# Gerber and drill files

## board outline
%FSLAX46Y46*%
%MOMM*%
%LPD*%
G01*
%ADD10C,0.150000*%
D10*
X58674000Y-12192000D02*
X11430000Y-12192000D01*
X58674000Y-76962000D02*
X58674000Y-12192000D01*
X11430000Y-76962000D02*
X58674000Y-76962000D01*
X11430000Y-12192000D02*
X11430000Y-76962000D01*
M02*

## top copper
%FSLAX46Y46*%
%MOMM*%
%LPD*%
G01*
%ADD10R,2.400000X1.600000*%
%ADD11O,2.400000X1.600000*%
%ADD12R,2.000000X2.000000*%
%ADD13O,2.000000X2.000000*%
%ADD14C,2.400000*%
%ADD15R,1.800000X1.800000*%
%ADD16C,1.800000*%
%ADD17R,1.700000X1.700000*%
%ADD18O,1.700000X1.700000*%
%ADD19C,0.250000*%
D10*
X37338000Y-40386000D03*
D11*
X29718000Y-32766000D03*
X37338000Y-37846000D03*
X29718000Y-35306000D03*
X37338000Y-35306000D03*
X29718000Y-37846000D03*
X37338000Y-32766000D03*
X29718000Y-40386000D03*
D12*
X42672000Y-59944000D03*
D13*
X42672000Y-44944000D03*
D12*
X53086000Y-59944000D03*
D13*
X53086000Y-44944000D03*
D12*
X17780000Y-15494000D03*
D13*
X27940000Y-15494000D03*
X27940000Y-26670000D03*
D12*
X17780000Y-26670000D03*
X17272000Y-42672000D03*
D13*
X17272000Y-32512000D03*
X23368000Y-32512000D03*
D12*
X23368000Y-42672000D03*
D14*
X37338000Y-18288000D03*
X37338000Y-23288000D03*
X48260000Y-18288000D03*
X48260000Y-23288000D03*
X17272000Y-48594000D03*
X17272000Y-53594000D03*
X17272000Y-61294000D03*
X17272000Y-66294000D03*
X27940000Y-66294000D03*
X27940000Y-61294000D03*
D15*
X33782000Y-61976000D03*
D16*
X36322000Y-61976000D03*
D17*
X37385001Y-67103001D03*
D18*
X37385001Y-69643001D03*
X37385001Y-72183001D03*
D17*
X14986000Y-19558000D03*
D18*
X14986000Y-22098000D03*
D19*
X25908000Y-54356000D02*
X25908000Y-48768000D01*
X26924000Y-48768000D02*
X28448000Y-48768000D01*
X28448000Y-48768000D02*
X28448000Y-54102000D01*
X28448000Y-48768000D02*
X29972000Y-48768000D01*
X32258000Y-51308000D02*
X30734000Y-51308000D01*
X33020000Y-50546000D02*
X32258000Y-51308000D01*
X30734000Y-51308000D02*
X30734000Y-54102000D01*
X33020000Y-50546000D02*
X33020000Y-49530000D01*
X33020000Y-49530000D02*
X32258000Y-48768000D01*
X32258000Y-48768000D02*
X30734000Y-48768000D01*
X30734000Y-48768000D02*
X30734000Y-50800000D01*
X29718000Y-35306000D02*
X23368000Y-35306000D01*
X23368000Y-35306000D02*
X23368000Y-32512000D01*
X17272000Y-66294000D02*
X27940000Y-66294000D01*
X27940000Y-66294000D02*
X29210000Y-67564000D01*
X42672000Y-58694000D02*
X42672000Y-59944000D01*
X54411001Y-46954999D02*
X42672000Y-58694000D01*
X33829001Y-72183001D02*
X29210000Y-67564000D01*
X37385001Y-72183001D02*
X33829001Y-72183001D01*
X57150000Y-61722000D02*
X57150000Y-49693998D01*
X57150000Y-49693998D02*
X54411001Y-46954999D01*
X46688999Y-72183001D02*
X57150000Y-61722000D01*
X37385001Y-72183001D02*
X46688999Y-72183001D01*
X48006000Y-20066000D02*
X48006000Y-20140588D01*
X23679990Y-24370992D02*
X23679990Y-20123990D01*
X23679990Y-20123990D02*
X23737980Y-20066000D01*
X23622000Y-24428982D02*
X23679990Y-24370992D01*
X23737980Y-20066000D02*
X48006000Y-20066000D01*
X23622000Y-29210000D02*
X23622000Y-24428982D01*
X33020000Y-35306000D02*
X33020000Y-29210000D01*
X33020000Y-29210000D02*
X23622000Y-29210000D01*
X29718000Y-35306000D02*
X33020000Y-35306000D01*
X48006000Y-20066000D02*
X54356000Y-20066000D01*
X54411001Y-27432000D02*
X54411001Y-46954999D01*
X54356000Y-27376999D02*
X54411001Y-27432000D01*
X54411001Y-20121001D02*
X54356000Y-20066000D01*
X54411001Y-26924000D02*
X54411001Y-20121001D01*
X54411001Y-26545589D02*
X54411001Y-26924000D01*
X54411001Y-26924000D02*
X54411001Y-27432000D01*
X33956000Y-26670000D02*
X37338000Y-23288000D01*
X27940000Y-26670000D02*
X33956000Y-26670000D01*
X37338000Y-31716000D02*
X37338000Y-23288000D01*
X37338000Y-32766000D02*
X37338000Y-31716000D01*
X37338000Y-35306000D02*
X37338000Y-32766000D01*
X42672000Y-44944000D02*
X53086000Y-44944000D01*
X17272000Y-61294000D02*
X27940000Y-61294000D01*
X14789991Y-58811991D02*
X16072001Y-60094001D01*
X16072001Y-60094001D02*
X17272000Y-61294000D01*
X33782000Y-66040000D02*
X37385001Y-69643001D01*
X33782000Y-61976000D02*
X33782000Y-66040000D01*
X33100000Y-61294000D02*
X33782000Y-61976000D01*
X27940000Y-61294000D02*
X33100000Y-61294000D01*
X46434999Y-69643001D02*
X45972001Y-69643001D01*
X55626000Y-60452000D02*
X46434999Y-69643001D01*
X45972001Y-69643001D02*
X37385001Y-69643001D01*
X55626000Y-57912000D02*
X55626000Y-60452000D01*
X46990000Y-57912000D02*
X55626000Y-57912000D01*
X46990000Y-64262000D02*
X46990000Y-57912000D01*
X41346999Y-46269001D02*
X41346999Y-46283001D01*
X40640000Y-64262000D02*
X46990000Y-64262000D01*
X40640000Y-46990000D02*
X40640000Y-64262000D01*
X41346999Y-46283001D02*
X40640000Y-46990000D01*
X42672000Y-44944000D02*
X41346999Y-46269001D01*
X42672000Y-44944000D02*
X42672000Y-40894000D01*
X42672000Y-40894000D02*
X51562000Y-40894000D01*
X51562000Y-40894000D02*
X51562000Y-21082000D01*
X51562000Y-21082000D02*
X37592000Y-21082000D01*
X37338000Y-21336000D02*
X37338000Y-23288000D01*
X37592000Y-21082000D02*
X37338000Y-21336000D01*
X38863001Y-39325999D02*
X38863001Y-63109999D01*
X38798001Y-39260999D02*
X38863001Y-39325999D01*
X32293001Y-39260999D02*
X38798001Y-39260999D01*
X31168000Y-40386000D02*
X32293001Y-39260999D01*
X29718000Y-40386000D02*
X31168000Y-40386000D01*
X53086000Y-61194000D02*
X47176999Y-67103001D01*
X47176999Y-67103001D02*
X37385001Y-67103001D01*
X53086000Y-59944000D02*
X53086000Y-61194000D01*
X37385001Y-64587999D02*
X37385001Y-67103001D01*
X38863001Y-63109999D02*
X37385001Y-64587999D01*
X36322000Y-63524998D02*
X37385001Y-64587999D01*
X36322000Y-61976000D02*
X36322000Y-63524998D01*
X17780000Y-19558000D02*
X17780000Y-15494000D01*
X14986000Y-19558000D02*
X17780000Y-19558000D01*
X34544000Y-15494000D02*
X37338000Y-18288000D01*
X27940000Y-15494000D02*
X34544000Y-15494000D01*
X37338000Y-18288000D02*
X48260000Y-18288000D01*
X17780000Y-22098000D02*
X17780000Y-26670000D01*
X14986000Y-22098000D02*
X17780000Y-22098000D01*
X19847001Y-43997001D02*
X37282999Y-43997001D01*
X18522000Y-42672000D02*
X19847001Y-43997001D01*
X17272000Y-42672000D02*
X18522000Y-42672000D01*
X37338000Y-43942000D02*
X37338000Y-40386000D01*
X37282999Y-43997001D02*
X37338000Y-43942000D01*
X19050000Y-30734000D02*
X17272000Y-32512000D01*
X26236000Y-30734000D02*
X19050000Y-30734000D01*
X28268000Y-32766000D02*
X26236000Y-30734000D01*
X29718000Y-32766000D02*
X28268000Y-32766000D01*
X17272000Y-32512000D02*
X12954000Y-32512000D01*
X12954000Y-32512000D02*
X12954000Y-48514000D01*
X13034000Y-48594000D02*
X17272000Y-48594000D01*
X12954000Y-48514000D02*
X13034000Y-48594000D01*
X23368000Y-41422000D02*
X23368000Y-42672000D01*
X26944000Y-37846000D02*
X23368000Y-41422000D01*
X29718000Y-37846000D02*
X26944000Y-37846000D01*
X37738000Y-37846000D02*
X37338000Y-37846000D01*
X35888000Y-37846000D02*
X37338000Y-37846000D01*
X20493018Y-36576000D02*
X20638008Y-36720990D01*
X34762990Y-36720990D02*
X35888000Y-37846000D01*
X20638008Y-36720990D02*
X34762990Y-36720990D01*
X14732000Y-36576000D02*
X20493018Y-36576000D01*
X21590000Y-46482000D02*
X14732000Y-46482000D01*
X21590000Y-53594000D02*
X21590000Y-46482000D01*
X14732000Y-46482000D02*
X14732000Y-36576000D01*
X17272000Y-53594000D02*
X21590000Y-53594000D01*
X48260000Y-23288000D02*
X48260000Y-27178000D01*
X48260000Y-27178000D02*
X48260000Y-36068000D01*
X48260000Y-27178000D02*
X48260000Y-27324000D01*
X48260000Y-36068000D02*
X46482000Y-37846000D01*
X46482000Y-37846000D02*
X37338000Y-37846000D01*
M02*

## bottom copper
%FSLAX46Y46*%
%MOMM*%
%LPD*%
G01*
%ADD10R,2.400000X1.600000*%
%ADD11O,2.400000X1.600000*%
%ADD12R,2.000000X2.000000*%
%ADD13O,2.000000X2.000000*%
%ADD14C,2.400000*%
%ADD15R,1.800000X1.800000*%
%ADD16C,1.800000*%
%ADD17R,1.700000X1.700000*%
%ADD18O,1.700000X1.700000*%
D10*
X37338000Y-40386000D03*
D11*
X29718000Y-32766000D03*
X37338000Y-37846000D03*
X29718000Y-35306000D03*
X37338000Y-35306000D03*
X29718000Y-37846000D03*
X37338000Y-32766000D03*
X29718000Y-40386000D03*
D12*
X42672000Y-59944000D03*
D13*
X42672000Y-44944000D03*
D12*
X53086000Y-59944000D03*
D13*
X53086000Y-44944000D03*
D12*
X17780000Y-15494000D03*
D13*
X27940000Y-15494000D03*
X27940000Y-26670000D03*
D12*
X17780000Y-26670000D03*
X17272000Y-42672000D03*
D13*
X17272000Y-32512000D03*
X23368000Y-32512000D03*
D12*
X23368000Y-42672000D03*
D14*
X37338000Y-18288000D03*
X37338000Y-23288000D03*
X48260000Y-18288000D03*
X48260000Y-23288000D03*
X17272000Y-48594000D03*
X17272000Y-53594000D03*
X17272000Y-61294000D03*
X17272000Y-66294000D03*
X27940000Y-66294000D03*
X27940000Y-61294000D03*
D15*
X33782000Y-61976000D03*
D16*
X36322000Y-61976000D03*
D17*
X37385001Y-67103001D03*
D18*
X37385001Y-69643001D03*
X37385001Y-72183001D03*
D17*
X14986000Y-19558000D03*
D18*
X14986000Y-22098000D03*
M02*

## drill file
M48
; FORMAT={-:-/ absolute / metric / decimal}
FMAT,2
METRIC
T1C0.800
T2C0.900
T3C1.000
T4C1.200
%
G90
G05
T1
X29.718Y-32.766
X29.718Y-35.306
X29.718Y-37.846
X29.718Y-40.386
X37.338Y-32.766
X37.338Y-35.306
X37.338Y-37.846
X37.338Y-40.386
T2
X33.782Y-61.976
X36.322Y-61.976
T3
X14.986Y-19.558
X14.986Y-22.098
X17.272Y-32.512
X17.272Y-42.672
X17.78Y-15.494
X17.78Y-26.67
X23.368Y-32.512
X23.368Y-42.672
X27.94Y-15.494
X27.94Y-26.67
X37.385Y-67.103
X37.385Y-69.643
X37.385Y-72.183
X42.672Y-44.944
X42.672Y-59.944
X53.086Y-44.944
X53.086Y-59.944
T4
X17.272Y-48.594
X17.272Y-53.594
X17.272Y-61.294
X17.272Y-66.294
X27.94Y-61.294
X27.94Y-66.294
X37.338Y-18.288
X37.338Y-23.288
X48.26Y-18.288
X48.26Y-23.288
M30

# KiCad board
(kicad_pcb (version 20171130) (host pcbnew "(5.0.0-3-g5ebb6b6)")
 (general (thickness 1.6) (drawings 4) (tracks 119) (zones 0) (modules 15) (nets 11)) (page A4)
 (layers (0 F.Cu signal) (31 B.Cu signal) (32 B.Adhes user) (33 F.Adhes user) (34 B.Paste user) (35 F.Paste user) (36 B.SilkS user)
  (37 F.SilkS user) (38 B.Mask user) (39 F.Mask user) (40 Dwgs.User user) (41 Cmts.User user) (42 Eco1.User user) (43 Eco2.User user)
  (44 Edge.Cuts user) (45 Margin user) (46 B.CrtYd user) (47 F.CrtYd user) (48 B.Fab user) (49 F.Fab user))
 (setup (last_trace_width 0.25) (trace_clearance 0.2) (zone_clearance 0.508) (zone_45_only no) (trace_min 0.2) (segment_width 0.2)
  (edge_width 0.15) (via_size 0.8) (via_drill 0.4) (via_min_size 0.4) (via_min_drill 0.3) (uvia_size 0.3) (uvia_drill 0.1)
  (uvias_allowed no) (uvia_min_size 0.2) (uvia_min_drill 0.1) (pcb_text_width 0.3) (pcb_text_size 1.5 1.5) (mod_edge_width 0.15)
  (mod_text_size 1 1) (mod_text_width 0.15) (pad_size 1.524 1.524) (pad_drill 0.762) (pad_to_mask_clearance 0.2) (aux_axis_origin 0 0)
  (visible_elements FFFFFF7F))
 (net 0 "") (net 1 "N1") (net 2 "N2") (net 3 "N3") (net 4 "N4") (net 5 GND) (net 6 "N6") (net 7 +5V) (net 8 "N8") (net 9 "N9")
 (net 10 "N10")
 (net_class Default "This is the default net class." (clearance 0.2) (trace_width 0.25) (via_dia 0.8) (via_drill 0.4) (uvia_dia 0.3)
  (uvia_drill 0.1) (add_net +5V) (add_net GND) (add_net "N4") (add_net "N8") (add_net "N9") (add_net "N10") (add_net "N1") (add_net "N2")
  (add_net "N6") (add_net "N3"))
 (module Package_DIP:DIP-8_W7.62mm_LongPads (layer F.Cu) (at 37.338 40.386 180)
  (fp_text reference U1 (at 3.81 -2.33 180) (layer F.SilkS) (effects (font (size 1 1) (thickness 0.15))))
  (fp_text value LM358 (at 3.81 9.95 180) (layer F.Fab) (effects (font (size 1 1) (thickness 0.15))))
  (pad 1 thru_hole rect (at 0 0 180) (size 2.4 1.6) (drill 0.8) (layers *.Cu *.Mask) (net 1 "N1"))
  (pad 5 thru_hole oval (at 7.62 7.62 180) (size 2.4 1.6) (drill 0.8) (layers *.Cu *.Mask) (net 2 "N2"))
  (pad 2 thru_hole oval (at 0 2.54 180) (size 2.4 1.6) (drill 0.8) (layers *.Cu *.Mask) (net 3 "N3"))
  (pad 6 thru_hole oval (at 7.62 5.08 180) (size 2.4 1.6) (drill 0.8) (layers *.Cu *.Mask) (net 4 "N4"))
  (pad 3 thru_hole oval (at 0 5.08 180) (size 2.4 1.6) (drill 0.8) (layers *.Cu *.Mask) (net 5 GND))
  (pad 7 thru_hole oval (at 7.62 2.54 180) (size 2.4 1.6) (drill 0.8) (layers *.Cu *.Mask) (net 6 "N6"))
  (pad 4 thru_hole oval (at 0 7.62 180) (size 2.4 1.6) (drill 0.8) (layers *.Cu *.Mask) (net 5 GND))
  (pad 8 thru_hole oval (at 7.62 0 180) (size 2.4 1.6) (drill 0.8) (layers *.Cu *.Mask) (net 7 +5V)))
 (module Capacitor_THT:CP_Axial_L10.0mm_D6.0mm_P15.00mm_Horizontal (layer F.Cu) (at 42.672 59.944 90)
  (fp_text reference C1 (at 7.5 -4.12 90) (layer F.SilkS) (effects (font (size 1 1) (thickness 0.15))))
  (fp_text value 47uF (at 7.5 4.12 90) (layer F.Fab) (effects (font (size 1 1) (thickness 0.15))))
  (pad 1 thru_hole rect (at 0 0 90) (size 2 2) (drill 1) (layers *.Cu *.Mask) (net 4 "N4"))
  (pad 2 thru_hole oval (at 15 0 90) (size 2 2) (drill 1) (layers *.Cu *.Mask) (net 5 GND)))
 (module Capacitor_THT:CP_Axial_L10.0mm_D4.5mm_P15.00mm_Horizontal (layer F.Cu) (at 53.086 59.944 90)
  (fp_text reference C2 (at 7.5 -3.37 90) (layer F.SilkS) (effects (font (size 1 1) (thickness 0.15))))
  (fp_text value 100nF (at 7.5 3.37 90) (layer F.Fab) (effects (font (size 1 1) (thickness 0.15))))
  (pad 1 thru_hole rect (at 0 0 90) (size 2 2) (drill 1) (layers *.Cu *.Mask) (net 7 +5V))
  (pad 2 thru_hole oval (at 15 0 90) (size 2 2) (drill 1) (layers *.Cu *.Mask) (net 5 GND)))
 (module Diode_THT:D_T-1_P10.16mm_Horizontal (layer F.Cu) (at 17.78 15.494)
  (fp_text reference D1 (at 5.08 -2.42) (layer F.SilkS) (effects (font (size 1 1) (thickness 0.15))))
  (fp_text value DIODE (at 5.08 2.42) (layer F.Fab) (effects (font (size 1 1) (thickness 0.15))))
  (pad 1 thru_hole rect (at 0 0) (size 2 2) (drill 1) (layers *.Cu *.Mask) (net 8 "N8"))
  (pad 2 thru_hole oval (at 10.16 0) (size 2 2) (drill 1) (layers *.Cu *.Mask) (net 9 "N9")))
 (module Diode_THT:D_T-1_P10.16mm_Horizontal (layer F.Cu) (at 17.78 26.67)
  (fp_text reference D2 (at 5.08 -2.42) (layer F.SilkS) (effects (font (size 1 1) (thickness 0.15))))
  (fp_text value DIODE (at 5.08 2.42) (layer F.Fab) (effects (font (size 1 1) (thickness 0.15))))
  (pad 2 thru_hole oval (at 10.16 0) (size 2 2) (drill 1) (layers *.Cu *.Mask) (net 5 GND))
  (pad 1 thru_hole rect (at 0 0) (size 2 2) (drill 1) (layers *.Cu *.Mask) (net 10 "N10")))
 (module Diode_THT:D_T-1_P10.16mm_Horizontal (layer F.Cu) (at 17.272 42.672 90)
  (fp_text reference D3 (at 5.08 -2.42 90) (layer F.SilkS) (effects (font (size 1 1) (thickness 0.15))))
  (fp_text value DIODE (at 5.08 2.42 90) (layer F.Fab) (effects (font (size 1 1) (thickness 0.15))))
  (pad 1 thru_hole rect (at 0 0 90) (size 2 2) (drill 1) (layers *.Cu *.Mask) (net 1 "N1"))
  (pad 2 thru_hole oval (at 10.16 0 90) (size 2 2) (drill 1) (layers *.Cu *.Mask) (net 2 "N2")))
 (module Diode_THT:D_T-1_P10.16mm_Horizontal (layer F.Cu) (at 23.368 42.672 90)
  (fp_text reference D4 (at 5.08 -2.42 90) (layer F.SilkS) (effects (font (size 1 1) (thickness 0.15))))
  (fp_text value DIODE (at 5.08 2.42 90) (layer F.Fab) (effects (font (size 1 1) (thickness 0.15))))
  (pad 2 thru_hole oval (at 10.16 0 90) (size 2 2) (drill 1) (layers *.Cu *.Mask) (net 4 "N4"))
  (pad 1 thru_hole rect (at 0 0 90) (size 2 2) (drill 1) (layers *.Cu *.Mask) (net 6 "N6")))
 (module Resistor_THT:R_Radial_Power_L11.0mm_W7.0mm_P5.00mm (layer F.Cu) (at 37.338 18.288 270)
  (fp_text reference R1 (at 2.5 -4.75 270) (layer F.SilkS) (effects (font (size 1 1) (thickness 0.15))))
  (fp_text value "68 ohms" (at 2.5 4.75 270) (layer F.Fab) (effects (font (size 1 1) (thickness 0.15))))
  (pad 1 thru_hole circle (at 0 0 270) (size 2.4 2.4) (drill 1.2) (layers *.Cu *.Mask) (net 9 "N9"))
  (pad 2 thru_hole circle (at 5 0 270) (size 2.4 2.4) (drill 1.2) (layers *.Cu *.Mask) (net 5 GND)))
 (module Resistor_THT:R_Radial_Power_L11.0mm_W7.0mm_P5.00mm (layer F.Cu) (at 48.26 23.288 90)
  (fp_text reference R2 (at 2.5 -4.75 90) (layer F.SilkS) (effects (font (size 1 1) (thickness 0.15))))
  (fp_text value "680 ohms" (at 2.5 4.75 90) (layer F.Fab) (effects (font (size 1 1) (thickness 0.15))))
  (pad 2 thru_hole circle (at 5 0 90) (size 2.4 2.4) (drill 1.2) (layers *.Cu *.Mask) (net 9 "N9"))
  (pad 1 thru_hole circle (at 0 0 90) (size 2.4 2.4) (drill 1.2) (layers *.Cu *.Mask) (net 3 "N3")))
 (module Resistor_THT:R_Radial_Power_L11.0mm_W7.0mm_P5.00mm (layer F.Cu) (at 17.272 48.594 270)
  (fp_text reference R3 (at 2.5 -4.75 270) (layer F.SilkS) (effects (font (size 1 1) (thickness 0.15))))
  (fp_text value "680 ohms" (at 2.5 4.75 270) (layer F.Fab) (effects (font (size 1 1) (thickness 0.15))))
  (pad 1 thru_hole circle (at 0 0 270) (size 2.4 2.4) (drill 1.2) (layers *.Cu *.Mask) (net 2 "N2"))
  (pad 2 thru_hole circle (at 5 0 270) (size 2.4 2.4) (drill 1.2) (layers *.Cu *.Mask) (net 3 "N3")))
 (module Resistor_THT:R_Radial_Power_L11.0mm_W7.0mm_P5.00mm (layer F.Cu) (at 17.272 66.294 90)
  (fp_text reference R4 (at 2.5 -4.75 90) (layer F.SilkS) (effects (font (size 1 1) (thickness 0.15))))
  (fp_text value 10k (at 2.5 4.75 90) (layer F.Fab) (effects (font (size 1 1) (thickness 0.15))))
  (pad 2 thru_hole circle (at 5 0 90) (size 2.4 2.4) (drill 1.2) (layers *.Cu *.Mask) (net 5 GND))
  (pad 1 thru_hole circle (at 0 0 90) (size 2.4 2.4) (drill 1.2) (layers *.Cu *.Mask) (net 4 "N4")))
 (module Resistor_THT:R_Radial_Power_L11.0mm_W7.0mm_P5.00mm (layer F.Cu) (at 27.94 66.294 90)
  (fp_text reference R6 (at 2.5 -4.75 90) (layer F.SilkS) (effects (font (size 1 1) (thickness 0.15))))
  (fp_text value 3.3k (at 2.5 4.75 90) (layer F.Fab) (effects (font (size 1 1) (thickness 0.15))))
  (pad 1 thru_hole circle (at 0 0 90) (size 2.4 2.4) (drill 1.2) (layers *.Cu *.Mask) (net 4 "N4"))
  (pad 2 thru_hole circle (at 5 0 90) (size 2.4 2.4) (drill 1.2) (layers *.Cu *.Mask) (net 5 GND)))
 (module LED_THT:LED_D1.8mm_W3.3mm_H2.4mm (layer F.Cu) (at 33.782 61.976)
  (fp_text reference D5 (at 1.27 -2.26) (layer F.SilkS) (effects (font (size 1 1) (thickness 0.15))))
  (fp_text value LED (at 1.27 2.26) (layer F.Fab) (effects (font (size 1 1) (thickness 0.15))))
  (pad 1 thru_hole rect (at 0 0) (size 1.8 1.8) (drill 0.9) (layers *.Cu *.Mask) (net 5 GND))
  (pad 2 thru_hole circle (at 2.54 0) (size 1.8 1.8) (drill 0.9) (layers *.Cu *.Mask) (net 7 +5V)))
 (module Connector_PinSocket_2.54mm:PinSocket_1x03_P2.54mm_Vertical (layer F.Cu) (at 37.385001 67.103001)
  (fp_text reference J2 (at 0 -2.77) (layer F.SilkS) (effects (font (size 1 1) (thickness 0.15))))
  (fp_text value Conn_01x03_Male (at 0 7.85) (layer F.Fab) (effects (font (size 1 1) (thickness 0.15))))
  (pad 1 thru_hole rect (at 0 0) (size 1.7 1.7) (drill 1) (layers *.Cu *.Mask) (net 7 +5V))
  (pad 2 thru_hole oval (at 0 2.54) (size 1.7 1.7) (drill 1) (layers *.Cu *.Mask) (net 5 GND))
  (pad 3 thru_hole oval (at 0 5.08) (size 1.7 1.7) (drill 1) (layers *.Cu *.Mask) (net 4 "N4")))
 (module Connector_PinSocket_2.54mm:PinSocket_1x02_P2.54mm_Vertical (layer F.Cu) (at 14.986 19.558)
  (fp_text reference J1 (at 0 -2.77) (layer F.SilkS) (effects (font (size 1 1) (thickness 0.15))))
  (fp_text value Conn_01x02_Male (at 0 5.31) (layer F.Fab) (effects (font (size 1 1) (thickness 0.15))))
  (pad 1 thru_hole rect (at 0 0) (size 1.7 1.7) (drill 1) (layers *.Cu *.Mask) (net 8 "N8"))
  (pad 2 thru_hole oval (at 0 2.54) (size 1.7 1.7) (drill 1) (layers *.Cu *.Mask) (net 10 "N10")))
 (gr_line (start 58.674 12.192) (end 11.43 12.192) (layer Edge.Cuts) (width 0.15))
 (gr_line (start 58.674 76.962) (end 58.674 12.192) (layer Edge.Cuts) (width 0.15))
 (gr_line (start 11.43 76.962) (end 58.674 76.962) (layer Edge.Cuts) (width 0.15))
 (gr_line (start 11.43 12.192) (end 11.43 76.962) (layer Edge.Cuts) (width 0.15))
 (segment (start 25.908 54.356) (end 25.908 48.768) (width 0.25) (layer F.Cu) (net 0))
 (segment (start 26.924 48.768) (end 28.448 48.768) (width 0.25) (layer F.Cu) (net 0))
 (segment (start 28.448 48.768) (end 28.448 54.102) (width 0.25) (layer F.Cu) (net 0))
 (segment (start 28.448 48.768) (end 29.972 48.768) (width 0.25) (layer F.Cu) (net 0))
 (segment (start 32.258 51.308) (end 30.734 51.308) (width 0.25) (layer F.Cu) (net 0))
 (segment (start 33.02 50.546) (end 32.258 51.308) (width 0.25) (layer F.Cu) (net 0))
 (segment (start 30.734 51.308) (end 30.734 54.102) (width 0.25) (layer F.Cu) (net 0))
 (segment (start 33.02 50.546) (end 33.02 49.53) (width 0.25) (layer F.Cu) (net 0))
 (segment (start 33.02 49.53) (end 32.258 48.768) (width 0.25) (layer F.Cu) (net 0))
 (segment (start 32.258 48.768) (end 30.734 48.768) (width 0.25) (layer F.Cu) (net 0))
 (segment (start 30.734 48.768) (end 30.734 50.8) (width 0.25) (layer F.Cu) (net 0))
 (segment (start 29.718 35.306) (end 23.368 35.306) (width 0.25) (layer F.Cu) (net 4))
 (segment (start 23.368 35.306) (end 23.368 32.512) (width 0.25) (layer F.Cu) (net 4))
 (segment (start 17.272 66.294) (end 27.94 66.294) (width 0.25) (layer F.Cu) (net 4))
 (segment (start 27.94 66.294) (end 29.21 67.564) (width 0.25) (layer F.Cu) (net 4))
 (segment (start 42.672 58.694) (end 42.672 59.944) (width 0.25) (layer F.Cu) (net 4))
 (segment (start 54.411001 46.954999) (end 42.672 58.694) (width 0.25) (layer F.Cu) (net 4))
 (segment (start 33.829001 72.183001) (end 29.21 67.564) (width 0.25) (layer F.Cu) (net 4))
 (segment (start 37.385001 72.183001) (end 33.829001 72.183001) (width 0.25) (layer F.Cu) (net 4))
 (segment (start 57.15 61.722) (end 57.15 49.693998) (width 0.25) (layer F.Cu) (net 4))
 (segment (start 57.15 49.693998) (end 54.411001 46.954999) (width 0.25) (layer F.Cu) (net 4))
 (segment (start 46.688999 72.183001) (end 57.15 61.722) (width 0.25) (layer F.Cu) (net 4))
 (segment (start 37.385001 72.183001) (end 46.688999 72.183001) (width 0.25) (layer F.Cu) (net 4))
 (segment (start 48.006 20.066) (end 48.006 20.140588) (width 0.25) (layer F.Cu) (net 4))
 (segment (start 23.67999 24.370992) (end 23.67999 20.12399) (width 0.25) (layer F.Cu) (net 4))
 (segment (start 23.67999 20.12399) (end 23.73798 20.066) (width 0.25) (layer F.Cu) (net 4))
 (segment (start 23.622 24.428982) (end 23.67999 24.370992) (width 0.25) (layer F.Cu) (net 4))
 (segment (start 23.73798 20.066) (end 48.006 20.066) (width 0.25) (layer F.Cu) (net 4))
 (segment (start 23.622 29.21) (end 23.622 24.428982) (width 0.25) (layer F.Cu) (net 4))
 (segment (start 33.02 35.306) (end 33.02 29.21) (width 0.25) (layer F.Cu) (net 4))
 (segment (start 33.02 29.21) (end 23.622 29.21) (width 0.25) (layer F.Cu) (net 4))
 (segment (start 29.718 35.306) (end 33.02 35.306) (width 0.25) (layer F.Cu) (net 4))
 (segment (start 48.006 20.066) (end 54.356 20.066) (width 0.25) (layer F.Cu) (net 4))
 (segment (start 54.411001 27.432) (end 54.411001 46.954999) (width 0.25) (layer F.Cu) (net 4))
 (segment (start 54.356 27.376999) (end 54.411001 27.432) (width 0.25) (layer F.Cu) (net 4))
 (segment (start 54.411001 20.121001) (end 54.356 20.066) (width 0.25) (layer F.Cu) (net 4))
 (segment (start 54.411001 26.924) (end 54.411001 20.121001) (width 0.25) (layer F.Cu) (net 4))
 (segment (start 54.411001 26.545589) (end 54.411001 26.924) (width 0.25) (layer F.Cu) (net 4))
 (segment (start 54.411001 26.924) (end 54.411001 27.432) (width 0.25) (layer F.Cu) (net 4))
 (segment (start 33.956 26.67) (end 37.338 23.288) (width 0.25) (layer F.Cu) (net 5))
 (segment (start 27.94 26.67) (end 33.956 26.67) (width 0.25) (layer F.Cu) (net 5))
 (segment (start 37.338 31.716) (end 37.338 23.288) (width 0.25) (layer F.Cu) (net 5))
 (segment (start 37.338 32.766) (end 37.338 31.716) (width 0.25) (layer F.Cu) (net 5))
 (segment (start 37.338 35.306) (end 37.338 32.766) (width 0.25) (layer F.Cu) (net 5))
 (segment (start 42.672 44.944) (end 53.086 44.944) (width 0.25) (layer F.Cu) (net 5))
 (segment (start 17.272 61.294) (end 27.94 61.294) (width 0.25) (layer F.Cu) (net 5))
 (segment (start 14.789991 58.811991) (end 16.072001 60.094001) (width 0.25) (layer F.Cu) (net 5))
 (segment (start 16.072001 60.094001) (end 17.272 61.294) (width 0.25) (layer F.Cu) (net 5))
 (segment (start 33.782 66.04) (end 37.385001 69.643001) (width 0.25) (layer F.Cu) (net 5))
 (segment (start 33.782 61.976) (end 33.782 66.04) (width 0.25) (layer F.Cu) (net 5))
 (segment (start 33.1 61.294) (end 33.782 61.976) (width 0.25) (layer F.Cu) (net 5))
 (segment (start 27.94 61.294) (end 33.1 61.294) (width 0.25) (layer F.Cu) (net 5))
 (segment (start 46.434999 69.643001) (end 45.972001 69.643001) (width 0.25) (layer F.Cu) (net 5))
 (segment (start 55.626 60.452) (end 46.434999 69.643001) (width 0.25) (layer F.Cu) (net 5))
 (segment (start 45.972001 69.643001) (end 37.385001 69.643001) (width 0.25) (layer F.Cu) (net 5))
 (segment (start 55.626 57.912) (end 55.626 60.452) (width 0.25) (layer F.Cu) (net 5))
 (segment (start 46.99 57.912) (end 55.626 57.912) (width 0.25) (layer F.Cu) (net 5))
 (segment (start 46.99 64.262) (end 46.99 57.912) (width 0.25) (layer F.Cu) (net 5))
 (segment (start 41.346999 46.269001) (end 41.346999 46.283001) (width 0.25) (layer F.Cu) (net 5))
 (segment (start 40.64 64.262) (end 46.99 64.262) (width 0.25) (layer F.Cu) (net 5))
 (segment (start 40.64 46.99) (end 40.64 64.262) (width 0.25) (layer F.Cu) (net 5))
 (segment (start 41.346999 46.283001) (end 40.64 46.99) (width 0.25) (layer F.Cu) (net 5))
 (segment (start 42.672 44.944) (end 41.346999 46.269001) (width 0.25) (layer F.Cu) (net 5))
 (segment (start 42.672 44.944) (end 42.672 40.894) (width 0.25) (layer F.Cu) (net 5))
 (segment (start 42.672 40.894) (end 51.562 40.894) (width 0.25) (layer F.Cu) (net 5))
 (segment (start 51.562 40.894) (end 51.562 21.082) (width 0.25) (layer F.Cu) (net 5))
 (segment (start 51.562 21.082) (end 37.592 21.082) (width 0.25) (layer F.Cu) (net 5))
 (segment (start 37.338 21.336) (end 37.338 23.288) (width 0.25) (layer F.Cu) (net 5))
 (segment (start 37.592 21.082) (end 37.338 21.336) (width 0.25) (layer F.Cu) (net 5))
 (segment (start 38.863001 39.325999) (end 38.863001 63.109999) (width 0.25) (layer F.Cu) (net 7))
 (segment (start 38.798001 39.260999) (end 38.863001 39.325999) (width 0.25) (layer F.Cu) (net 7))
 (segment (start 32.293001 39.260999) (end 38.798001 39.260999) (width 0.25) (layer F.Cu) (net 7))
 (segment (start 31.168 40.386) (end 32.293001 39.260999) (width 0.25) (layer F.Cu) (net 7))
 (segment (start 29.718 40.386) (end 31.168 40.386) (width 0.25) (layer F.Cu) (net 7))
 (segment (start 53.086 61.194) (end 47.176999 67.103001) (width 0.25) (layer F.Cu) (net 7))
 (segment (start 47.176999 67.103001) (end 37.385001 67.103001) (width 0.25) (layer F.Cu) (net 7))
 (segment (start 53.086 59.944) (end 53.086 61.194) (width 0.25) (layer F.Cu) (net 7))
 (segment (start 37.385001 64.587999) (end 37.385001 67.103001) (width 0.25) (layer F.Cu) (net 7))
 (segment (start 38.863001 63.109999) (end 37.385001 64.587999) (width 0.25) (layer F.Cu) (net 7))
 (segment (start 36.322 63.524998) (end 37.385001 64.587999) (width 0.25) (layer F.Cu) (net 7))
 (segment (start 36.322 61.976) (end 36.322 63.524998) (width 0.25) (layer F.Cu) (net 7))
 (segment (start 17.78 19.558) (end 17.78 15.494) (width 0.25) (layer F.Cu) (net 8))
 (segment (start 14.986 19.558) (end 17.78 19.558) (width 0.25) (layer F.Cu) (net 8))
 (segment (start 34.544 15.494) (end 37.338 18.288) (width 0.25) (layer F.Cu) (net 9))
 (segment (start 27.94 15.494) (end 34.544 15.494) (width 0.25) (layer F.Cu) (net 9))
 (segment (start 37.338 18.288) (end 48.26 18.288) (width 0.25) (layer F.Cu) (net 9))
 (segment (start 17.78 22.098) (end 17.78 26.67) (width 0.25) (layer F.Cu) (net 10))
 (segment (start 14.986 22.098) (end 17.78 22.098) (width 0.25) (layer F.Cu) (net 10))
 (segment (start 19.847001 43.997001) (end 37.282999 43.997001) (width 0.25) (layer F.Cu) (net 1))
 (segment (start 18.522 42.672) (end 19.847001 43.997001) (width 0.25) (layer F.Cu) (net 1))
 (segment (start 17.272 42.672) (end 18.522 42.672) (width 0.25) (layer F.Cu) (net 1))
 (segment (start 37.338 43.942) (end 37.338 40.386) (width 0.25) (layer F.Cu) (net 1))
 (segment (start 37.282999 43.997001) (end 37.338 43.942) (width 0.25) (layer F.Cu) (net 1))
 (segment (start 19.05 30.734) (end 17.272 32.512) (width 0.25) (layer F.Cu) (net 2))
 (segment (start 26.236 30.734) (end 19.05 30.734) (width 0.25) (layer F.Cu) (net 2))
 (segment (start 28.268 32.766) (end 26.236 30.734) (width 0.25) (layer F.Cu) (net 2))
 (segment (start 29.718 32.766) (end 28.268 32.766) (width 0.25) (layer F.Cu) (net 2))
 (segment (start 17.272 32.512) (end 12.954 32.512) (width 0.25) (layer F.Cu) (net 2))
 (segment (start 12.954 32.512) (end 12.954 48.514) (width 0.25) (layer F.Cu) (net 2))
 (segment (start 13.034 48.594) (end 17.272 48.594) (width 0.25) (layer F.Cu) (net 2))
 (segment (start 12.954 48.514) (end 13.034 48.594) (width 0.25) (layer F.Cu) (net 2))
 (segment (start 23.368 41.422) (end 23.368 42.672) (width 0.25) (layer F.Cu) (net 6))
 (segment (start 26.944 37.846) (end 23.368 41.422) (width 0.25) (layer F.Cu) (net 6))
 (segment (start 29.718 37.846) (end 26.944 37.846) (width 0.25) (layer F.Cu) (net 6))
 (segment (start 37.738 37.846) (end 37.338 37.846) (width 0.25) (layer F.Cu) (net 3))
 (segment (start 35.888 37.846) (end 37.338 37.846) (width 0.25) (layer F.Cu) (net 3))
 (segment (start 20.493018 36.576) (end 20.638008 36.72099) (width 0.25) (layer F.Cu) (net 3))
 (segment (start 34.76299 36.72099) (end 35.888 37.846) (width 0.25) (layer F.Cu) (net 3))
 (segment (start 20.638008 36.72099) (end 34.76299 36.72099) (width 0.25) (layer F.Cu) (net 3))
 (segment (start 14.732 36.576) (end 20.493018 36.576) (width 0.25) (layer F.Cu) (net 3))
 (segment (start 21.59 46.482) (end 14.732 46.482) (width 0.25) (layer F.Cu) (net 3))
 (segment (start 21.59 53.594) (end 21.59 46.482) (width 0.25) (layer F.Cu) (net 3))
 (segment (start 14.732 46.482) (end 14.732 36.576) (width 0.25) (layer F.Cu) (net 3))
 (segment (start 17.272 53.594) (end 21.59 53.594) (width 0.25) (layer F.Cu) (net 3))
 (segment (start 48.26 23.288) (end 48.26 27.178) (width 0.25) (layer F.Cu) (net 3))
 (segment (start 48.26 27.178) (end 48.26 36.068) (width 0.25) (layer F.Cu) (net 3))
 (segment (start 48.26 27.178) (end 48.26 27.324) (width 0.25) (layer F.Cu) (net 3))
 (segment (start 48.26 36.068) (end 46.482 37.846) (width 0.25) (layer F.Cu) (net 3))
 (segment (start 46.482 37.846) (end 37.338 37.846) (width 0.25) (layer F.Cu) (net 3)))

